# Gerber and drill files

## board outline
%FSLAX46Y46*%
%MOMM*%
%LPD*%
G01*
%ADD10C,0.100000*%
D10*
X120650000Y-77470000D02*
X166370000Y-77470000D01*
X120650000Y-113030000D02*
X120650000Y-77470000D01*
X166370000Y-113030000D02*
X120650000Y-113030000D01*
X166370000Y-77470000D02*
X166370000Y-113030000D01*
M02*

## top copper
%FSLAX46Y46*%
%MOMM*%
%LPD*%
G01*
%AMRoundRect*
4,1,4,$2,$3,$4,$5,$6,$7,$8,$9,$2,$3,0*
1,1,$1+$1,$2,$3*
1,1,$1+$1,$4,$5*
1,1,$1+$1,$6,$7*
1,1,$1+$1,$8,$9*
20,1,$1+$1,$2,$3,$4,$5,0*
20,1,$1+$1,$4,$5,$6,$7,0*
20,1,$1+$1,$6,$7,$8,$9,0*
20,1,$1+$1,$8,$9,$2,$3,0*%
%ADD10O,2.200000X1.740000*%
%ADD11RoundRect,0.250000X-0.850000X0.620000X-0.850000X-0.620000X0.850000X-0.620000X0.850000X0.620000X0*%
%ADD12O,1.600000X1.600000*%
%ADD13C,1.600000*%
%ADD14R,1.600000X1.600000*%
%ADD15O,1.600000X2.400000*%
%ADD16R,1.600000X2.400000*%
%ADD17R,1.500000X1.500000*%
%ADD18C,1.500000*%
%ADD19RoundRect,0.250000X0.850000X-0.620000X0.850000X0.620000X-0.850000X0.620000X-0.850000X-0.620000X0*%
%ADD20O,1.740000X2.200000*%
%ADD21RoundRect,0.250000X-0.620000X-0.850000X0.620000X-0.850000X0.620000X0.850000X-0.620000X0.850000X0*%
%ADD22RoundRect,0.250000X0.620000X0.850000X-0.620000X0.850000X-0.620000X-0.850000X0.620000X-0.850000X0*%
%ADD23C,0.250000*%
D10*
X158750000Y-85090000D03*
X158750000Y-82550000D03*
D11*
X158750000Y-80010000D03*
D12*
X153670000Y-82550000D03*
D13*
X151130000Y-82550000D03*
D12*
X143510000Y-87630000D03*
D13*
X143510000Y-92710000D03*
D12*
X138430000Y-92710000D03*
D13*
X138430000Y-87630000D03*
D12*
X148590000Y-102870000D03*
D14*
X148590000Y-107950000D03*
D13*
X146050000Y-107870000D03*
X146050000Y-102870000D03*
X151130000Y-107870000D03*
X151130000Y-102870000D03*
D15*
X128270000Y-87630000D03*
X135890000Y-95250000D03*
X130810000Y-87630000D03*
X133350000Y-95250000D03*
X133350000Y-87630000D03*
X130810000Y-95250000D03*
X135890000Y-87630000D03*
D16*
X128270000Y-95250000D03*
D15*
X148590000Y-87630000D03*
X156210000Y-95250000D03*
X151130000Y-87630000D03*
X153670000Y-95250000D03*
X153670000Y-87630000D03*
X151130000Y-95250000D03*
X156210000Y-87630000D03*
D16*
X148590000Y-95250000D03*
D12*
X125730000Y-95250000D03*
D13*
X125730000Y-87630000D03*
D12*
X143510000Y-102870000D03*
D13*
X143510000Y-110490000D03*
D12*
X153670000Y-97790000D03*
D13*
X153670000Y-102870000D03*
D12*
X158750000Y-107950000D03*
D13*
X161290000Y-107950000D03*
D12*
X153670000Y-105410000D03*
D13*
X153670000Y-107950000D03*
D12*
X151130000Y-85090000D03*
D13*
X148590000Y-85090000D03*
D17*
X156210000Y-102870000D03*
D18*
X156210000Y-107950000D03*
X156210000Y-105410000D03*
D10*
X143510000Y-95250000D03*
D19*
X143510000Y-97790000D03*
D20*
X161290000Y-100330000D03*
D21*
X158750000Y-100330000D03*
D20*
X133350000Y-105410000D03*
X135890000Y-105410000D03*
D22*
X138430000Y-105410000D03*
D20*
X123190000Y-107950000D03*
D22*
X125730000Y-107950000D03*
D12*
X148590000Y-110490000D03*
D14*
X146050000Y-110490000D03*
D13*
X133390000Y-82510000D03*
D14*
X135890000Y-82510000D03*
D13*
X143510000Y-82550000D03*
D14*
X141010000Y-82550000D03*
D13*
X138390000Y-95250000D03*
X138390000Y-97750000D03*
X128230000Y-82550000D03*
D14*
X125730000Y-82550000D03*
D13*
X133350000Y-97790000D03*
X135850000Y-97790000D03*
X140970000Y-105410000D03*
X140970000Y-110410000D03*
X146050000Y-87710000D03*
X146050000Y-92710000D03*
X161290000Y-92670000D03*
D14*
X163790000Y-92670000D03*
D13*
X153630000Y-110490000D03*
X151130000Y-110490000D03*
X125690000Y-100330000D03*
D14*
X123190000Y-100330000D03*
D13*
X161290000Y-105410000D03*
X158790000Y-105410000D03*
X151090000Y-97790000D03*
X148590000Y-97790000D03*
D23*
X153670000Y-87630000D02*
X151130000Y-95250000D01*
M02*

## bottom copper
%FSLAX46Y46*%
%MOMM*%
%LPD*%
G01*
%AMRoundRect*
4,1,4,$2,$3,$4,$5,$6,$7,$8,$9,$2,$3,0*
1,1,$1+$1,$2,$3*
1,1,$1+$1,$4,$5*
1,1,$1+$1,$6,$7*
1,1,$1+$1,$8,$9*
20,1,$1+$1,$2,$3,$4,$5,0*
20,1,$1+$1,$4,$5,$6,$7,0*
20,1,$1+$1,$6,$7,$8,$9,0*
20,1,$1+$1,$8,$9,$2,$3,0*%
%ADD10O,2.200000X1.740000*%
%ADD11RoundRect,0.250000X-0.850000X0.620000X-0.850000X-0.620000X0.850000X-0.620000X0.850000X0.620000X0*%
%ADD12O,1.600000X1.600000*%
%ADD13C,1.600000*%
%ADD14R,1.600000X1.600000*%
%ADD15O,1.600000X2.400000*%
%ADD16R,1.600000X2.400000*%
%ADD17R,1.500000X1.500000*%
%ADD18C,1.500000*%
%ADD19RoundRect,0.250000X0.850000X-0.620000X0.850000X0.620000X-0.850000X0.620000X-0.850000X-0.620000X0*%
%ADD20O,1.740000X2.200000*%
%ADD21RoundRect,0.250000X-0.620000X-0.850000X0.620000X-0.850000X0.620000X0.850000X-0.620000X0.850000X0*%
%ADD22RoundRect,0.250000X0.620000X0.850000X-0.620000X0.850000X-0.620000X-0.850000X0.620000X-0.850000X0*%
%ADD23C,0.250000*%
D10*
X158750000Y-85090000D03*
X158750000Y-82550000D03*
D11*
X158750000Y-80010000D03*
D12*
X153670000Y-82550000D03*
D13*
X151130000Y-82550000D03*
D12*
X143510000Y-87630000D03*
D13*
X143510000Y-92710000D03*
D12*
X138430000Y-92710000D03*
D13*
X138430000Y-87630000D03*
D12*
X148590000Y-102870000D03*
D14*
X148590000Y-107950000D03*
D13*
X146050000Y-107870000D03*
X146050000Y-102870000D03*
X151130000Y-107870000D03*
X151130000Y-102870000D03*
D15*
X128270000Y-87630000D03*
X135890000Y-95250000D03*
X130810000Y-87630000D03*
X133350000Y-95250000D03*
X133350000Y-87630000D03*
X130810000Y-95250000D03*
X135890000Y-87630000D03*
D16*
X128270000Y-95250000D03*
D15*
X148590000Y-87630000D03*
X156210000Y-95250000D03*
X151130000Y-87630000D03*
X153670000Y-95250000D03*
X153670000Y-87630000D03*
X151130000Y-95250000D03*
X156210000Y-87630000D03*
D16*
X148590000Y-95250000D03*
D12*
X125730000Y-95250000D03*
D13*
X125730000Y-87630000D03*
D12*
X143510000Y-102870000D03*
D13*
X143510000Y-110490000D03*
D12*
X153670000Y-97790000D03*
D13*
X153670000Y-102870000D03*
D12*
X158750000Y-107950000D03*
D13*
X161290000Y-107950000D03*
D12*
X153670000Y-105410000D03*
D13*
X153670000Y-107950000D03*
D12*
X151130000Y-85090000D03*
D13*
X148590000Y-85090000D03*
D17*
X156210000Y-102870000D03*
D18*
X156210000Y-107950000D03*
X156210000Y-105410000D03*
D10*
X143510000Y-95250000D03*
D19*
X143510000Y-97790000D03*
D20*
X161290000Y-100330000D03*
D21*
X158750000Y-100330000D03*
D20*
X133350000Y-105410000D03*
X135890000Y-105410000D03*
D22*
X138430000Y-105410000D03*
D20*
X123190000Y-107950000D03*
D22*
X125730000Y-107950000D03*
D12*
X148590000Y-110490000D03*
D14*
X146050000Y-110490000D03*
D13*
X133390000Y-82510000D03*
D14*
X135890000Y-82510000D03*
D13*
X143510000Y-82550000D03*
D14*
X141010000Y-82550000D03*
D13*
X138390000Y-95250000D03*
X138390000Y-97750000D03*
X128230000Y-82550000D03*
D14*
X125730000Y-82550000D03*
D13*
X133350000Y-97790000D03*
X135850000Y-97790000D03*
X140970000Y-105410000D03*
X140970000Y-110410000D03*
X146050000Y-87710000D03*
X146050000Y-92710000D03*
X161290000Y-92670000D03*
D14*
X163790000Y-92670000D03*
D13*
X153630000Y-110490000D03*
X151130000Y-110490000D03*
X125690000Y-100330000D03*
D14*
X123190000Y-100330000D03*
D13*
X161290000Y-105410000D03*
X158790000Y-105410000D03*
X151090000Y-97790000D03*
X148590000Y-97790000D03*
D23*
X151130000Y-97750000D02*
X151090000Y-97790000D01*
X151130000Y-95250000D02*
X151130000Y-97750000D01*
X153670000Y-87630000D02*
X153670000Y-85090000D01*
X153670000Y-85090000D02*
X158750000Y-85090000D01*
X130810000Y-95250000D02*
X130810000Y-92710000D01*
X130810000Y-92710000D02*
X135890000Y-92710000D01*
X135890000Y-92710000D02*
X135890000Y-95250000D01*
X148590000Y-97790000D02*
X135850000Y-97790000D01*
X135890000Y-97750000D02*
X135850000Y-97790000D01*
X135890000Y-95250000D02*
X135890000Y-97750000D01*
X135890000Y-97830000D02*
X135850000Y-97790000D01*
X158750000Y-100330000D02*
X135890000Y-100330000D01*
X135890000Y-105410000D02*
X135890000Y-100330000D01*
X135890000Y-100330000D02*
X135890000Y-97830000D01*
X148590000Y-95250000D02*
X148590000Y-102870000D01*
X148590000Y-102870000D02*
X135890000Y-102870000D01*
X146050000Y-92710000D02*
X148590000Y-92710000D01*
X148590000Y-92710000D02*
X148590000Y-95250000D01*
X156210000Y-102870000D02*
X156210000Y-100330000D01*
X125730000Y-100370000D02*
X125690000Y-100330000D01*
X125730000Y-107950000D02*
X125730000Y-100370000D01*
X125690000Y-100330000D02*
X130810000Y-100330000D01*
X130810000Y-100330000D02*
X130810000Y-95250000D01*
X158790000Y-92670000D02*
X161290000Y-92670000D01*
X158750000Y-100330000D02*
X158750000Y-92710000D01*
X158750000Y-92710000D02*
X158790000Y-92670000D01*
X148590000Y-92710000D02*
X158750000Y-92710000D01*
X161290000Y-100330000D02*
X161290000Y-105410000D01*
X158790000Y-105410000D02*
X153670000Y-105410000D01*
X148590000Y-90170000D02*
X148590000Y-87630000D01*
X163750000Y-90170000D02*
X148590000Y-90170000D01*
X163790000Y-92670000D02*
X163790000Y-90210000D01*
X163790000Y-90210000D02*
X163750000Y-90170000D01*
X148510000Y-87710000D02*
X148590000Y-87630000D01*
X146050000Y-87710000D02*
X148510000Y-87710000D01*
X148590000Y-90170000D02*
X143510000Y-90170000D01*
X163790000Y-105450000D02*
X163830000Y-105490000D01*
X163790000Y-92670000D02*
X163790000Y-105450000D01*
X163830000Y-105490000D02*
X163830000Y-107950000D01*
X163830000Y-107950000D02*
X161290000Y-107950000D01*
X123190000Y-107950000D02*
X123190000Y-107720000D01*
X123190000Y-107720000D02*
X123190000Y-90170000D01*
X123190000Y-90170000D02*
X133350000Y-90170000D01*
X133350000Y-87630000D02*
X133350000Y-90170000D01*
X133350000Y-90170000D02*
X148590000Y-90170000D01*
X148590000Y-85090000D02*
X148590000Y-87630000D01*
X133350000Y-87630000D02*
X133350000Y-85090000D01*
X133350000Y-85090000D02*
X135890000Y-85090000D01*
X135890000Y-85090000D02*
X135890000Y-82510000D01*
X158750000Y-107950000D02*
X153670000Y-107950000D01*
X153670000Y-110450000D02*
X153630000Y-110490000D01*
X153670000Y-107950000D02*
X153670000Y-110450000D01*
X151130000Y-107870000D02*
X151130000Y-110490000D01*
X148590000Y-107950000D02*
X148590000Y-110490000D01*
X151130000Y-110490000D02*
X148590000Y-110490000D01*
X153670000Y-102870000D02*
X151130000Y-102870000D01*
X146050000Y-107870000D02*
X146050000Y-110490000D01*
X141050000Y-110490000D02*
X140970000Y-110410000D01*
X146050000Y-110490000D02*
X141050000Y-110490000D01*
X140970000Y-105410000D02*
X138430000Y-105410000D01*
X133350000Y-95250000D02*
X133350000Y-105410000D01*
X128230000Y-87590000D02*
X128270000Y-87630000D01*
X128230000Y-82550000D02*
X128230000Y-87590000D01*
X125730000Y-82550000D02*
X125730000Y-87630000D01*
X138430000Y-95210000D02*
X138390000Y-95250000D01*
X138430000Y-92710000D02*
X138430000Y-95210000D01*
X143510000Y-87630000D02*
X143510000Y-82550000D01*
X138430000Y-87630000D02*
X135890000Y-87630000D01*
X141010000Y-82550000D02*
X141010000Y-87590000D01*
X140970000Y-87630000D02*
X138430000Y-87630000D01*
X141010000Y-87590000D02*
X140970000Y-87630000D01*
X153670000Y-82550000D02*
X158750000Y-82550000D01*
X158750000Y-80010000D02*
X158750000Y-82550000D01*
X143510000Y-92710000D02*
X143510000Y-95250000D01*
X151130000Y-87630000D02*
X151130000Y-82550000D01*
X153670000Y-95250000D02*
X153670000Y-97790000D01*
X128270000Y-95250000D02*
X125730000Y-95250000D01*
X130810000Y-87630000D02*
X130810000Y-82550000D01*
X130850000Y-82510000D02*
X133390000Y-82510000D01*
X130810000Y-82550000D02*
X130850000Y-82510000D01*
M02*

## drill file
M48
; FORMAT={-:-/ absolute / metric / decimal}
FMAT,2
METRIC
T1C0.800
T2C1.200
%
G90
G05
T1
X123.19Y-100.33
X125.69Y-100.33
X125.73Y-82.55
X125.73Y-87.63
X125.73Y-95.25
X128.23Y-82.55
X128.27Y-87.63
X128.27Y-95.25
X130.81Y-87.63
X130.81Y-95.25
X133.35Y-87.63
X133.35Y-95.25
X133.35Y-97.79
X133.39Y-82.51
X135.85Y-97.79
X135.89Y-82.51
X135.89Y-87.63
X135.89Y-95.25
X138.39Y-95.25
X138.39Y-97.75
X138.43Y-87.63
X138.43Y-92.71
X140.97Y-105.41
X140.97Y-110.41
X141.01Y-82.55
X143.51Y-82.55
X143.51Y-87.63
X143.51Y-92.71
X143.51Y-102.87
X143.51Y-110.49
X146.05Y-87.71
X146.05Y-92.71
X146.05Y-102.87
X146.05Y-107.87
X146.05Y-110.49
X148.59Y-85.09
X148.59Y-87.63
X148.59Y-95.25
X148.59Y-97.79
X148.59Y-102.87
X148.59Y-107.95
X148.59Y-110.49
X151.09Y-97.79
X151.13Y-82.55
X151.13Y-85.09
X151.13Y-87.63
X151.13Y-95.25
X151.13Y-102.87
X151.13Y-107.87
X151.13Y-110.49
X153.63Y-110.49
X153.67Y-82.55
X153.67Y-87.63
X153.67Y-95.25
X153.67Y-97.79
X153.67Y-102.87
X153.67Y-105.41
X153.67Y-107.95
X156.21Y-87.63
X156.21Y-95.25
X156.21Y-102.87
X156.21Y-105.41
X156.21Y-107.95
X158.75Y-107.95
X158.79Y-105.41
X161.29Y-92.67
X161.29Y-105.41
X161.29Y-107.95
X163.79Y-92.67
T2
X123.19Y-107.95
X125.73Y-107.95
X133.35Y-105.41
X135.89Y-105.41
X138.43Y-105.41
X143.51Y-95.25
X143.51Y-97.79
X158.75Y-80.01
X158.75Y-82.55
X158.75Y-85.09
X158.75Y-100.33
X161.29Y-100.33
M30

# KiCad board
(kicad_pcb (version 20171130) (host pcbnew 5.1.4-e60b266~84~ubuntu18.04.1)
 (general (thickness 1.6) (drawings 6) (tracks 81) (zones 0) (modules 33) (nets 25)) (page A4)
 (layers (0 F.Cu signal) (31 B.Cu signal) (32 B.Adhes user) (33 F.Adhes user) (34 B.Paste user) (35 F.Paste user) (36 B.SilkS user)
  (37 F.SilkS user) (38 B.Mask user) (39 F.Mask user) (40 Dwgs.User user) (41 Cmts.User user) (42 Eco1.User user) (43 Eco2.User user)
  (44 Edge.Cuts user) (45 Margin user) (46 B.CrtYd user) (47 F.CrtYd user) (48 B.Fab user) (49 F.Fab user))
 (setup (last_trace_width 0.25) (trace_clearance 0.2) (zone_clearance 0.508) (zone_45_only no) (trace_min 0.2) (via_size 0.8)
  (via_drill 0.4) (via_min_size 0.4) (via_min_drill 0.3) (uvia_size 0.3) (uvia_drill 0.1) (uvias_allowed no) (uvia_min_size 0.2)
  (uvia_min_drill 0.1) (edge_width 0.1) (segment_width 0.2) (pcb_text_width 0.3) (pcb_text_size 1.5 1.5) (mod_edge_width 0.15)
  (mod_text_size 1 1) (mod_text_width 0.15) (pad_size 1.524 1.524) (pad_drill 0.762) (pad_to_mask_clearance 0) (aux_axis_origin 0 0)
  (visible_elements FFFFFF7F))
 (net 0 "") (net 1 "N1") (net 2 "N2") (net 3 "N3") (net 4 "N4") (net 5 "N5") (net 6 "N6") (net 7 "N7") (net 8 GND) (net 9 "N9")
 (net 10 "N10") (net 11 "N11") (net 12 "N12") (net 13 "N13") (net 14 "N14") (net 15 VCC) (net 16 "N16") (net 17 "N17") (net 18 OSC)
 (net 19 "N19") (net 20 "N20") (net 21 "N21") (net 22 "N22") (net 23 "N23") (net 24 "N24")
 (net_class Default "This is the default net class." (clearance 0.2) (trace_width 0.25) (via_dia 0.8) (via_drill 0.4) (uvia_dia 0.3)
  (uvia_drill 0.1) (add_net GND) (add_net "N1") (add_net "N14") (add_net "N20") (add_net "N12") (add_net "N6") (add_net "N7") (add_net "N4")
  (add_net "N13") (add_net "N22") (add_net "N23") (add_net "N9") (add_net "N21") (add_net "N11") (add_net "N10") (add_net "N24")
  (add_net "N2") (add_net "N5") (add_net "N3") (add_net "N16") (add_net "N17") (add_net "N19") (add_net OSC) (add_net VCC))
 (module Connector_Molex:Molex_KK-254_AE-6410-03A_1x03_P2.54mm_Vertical (layer F.Cu) (at 158.75 80.01 270)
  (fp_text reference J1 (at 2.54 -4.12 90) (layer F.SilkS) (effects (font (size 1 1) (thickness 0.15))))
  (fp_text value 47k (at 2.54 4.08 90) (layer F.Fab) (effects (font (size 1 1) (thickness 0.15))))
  (pad 3 thru_hole oval (at 5.08 0 270) (size 1.74 2.2) (drill 1.2) (layers *.Cu *.Mask) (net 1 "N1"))
  (pad 2 thru_hole oval (at 2.54 0 270) (size 1.74 2.2) (drill 1.2) (layers *.Cu *.Mask) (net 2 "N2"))
  (pad 1 thru_hole roundrect (at 0 0 270) (size 1.74 2.2) (drill 1.2) (layers *.Cu *.Mask) (roundrect_rratio 0.143678) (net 2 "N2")))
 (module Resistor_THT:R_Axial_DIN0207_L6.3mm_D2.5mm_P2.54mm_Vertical (layer F.Cu) (at 151.13 82.55)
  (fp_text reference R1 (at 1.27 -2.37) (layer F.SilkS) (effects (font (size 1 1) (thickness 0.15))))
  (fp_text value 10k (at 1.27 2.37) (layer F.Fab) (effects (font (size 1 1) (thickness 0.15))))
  (pad 2 thru_hole oval (at 2.54 0) (size 1.6 1.6) (drill 0.8) (layers *.Cu *.Mask) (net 2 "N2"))
  (pad 1 thru_hole circle (at 0 0) (size 1.6 1.6) (drill 0.8) (layers *.Cu *.Mask) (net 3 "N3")))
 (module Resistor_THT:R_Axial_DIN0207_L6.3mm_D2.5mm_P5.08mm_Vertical (layer F.Cu) (at 143.51 92.71 90)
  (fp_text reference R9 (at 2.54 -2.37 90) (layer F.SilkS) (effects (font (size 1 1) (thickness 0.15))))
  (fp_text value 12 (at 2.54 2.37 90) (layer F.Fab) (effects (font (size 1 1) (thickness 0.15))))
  (pad 2 thru_hole oval (at 5.08 0 90) (size 1.6 1.6) (drill 0.8) (layers *.Cu *.Mask) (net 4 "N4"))
  (pad 1 thru_hole circle (at 0 0 90) (size 1.6 1.6) (drill 0.8) (layers *.Cu *.Mask) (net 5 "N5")))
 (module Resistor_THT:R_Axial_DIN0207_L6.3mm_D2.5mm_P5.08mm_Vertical (layer F.Cu) (at 138.43 87.63 270)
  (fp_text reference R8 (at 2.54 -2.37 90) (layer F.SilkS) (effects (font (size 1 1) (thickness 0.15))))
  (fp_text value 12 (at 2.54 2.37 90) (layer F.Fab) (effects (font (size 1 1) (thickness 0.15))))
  (pad 2 thru_hole oval (at 5.08 0 270) (size 1.6 1.6) (drill 0.8) (layers *.Cu *.Mask) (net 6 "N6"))
  (pad 1 thru_hole circle (at 0 0 270) (size 1.6 1.6) (drill 0.8) (layers *.Cu *.Mask) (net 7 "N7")))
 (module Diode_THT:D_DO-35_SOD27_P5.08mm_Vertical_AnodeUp (layer F.Cu) (at 148.59 107.95 90)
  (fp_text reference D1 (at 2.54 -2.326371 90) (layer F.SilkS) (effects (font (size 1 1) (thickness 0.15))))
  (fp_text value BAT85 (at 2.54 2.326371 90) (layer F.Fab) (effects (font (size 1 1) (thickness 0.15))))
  (pad 2 thru_hole oval (at 5.08 0 90) (size 1.6 1.6) (drill 0.8) (layers *.Cu *.Mask) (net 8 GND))
  (pad 1 thru_hole rect (at 0 0 90) (size 1.6 1.6) (drill 0.8) (layers *.Cu *.Mask) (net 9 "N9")))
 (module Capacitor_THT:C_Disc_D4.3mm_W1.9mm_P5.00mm (layer F.Cu) (at 146.05 102.87 270)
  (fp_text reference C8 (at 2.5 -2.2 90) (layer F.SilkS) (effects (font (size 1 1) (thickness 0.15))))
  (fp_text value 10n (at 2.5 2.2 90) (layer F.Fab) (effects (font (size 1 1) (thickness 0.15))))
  (pad 2 thru_hole circle (at 5 0 270) (size 1.6 1.6) (drill 0.8) (layers *.Cu *.Mask) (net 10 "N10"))
  (pad 1 thru_hole circle (at 0 0 270) (size 1.6 1.6) (drill 0.8) (layers *.Cu *.Mask) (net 8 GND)))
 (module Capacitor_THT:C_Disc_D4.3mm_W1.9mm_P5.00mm (layer F.Cu) (at 151.13 102.87 270)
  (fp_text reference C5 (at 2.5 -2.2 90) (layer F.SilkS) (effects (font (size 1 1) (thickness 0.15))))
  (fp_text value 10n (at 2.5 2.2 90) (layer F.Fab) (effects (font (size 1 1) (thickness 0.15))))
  (pad 2 thru_hole circle (at 5 0 270) (size 1.6 1.6) (drill 0.8) (layers *.Cu *.Mask) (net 9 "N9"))
  (pad 1 thru_hole circle (at 0 0 270) (size 1.6 1.6) (drill 0.8) (layers *.Cu *.Mask) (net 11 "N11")))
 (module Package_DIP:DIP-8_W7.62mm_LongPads (layer F.Cu) (at 128.27 95.25 90)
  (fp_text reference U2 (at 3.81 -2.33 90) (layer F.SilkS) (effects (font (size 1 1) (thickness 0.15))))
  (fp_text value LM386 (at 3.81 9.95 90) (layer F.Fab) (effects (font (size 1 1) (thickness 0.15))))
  (pad 8 thru_hole oval (at 7.62 0 90) (size 2.4 1.6) (drill 0.8) (layers *.Cu *.Mask) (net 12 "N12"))
  (pad 4 thru_hole oval (at 0 7.62 90) (size 2.4 1.6) (drill 0.8) (layers *.Cu *.Mask) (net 8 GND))
  (pad 7 thru_hole oval (at 7.62 2.54 90) (size 2.4 1.6) (drill 0.8) (layers *.Cu *.Mask) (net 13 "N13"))
  (pad 3 thru_hole oval (at 0 5.08 90) (size 2.4 1.6) (drill 0.8) (layers *.Cu *.Mask) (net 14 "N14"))
  (pad 6 thru_hole oval (at 7.62 5.08 90) (size 2.4 1.6) (drill 0.8) (layers *.Cu *.Mask) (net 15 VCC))
  (pad 2 thru_hole oval (at 0 2.54 90) (size 2.4 1.6) (drill 0.8) (layers *.Cu *.Mask) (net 8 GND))
  (pad 5 thru_hole oval (at 7.62 7.62 90) (size 2.4 1.6) (drill 0.8) (layers *.Cu *.Mask) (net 7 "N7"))
  (pad 1 thru_hole rect (at 0 0 90) (size 2.4 1.6) (drill 0.8) (layers *.Cu *.Mask) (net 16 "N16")))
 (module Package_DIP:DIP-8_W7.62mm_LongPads (layer F.Cu) (at 148.59 95.25 90)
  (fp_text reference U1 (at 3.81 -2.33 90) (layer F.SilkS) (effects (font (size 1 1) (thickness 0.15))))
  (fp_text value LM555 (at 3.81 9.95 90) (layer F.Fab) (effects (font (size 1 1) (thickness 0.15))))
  (pad 8 thru_hole oval (at 7.62 0 90) (size 2.4 1.6) (drill 0.8) (layers *.Cu *.Mask) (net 15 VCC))
  (pad 4 thru_hole oval (at 0 7.62 90) (size 2.4 1.6) (drill 0.8) (layers *.Cu *.Mask) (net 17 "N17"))
  (pad 7 thru_hole oval (at 7.62 2.54 90) (size 2.4 1.6) (drill 0.8) (layers *.Cu *.Mask) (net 3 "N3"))
  (pad 3 thru_hole oval (at 0 5.08 90) (size 2.4 1.6) (drill 0.8) (layers *.Cu *.Mask) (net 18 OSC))
  (pad 6 thru_hole oval (at 7.62 5.08 90) (size 2.4 1.6) (drill 0.8) (layers *.Cu *.Mask) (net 1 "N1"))
  (pad 2 thru_hole oval (at 0 2.54 90) (size 2.4 1.6) (drill 0.8) (layers *.Cu *.Mask) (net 1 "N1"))
  (pad 5 thru_hole oval (at 7.62 7.62 90) (size 2.4 1.6) (drill 0.8) (layers *.Cu *.Mask) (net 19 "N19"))
  (pad 1 thru_hole rect (at 0 0 90) (size 2.4 1.6) (drill 0.8) (layers *.Cu *.Mask) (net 8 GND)))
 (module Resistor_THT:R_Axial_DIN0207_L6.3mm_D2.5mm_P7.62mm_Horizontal (layer F.Cu) (at 125.73 87.63 270)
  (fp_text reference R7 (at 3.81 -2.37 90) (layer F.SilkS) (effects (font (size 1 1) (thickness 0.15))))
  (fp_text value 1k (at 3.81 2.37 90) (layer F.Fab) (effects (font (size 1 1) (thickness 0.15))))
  (pad 2 thru_hole oval (at 7.62 0 270) (size 1.6 1.6) (drill 0.8) (layers *.Cu *.Mask) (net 16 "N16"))
  (pad 1 thru_hole circle (at 0 0 270) (size 1.6 1.6) (drill 0.8) (layers *.Cu *.Mask) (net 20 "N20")))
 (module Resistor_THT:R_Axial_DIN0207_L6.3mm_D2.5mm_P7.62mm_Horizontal (layer F.Cu) (at 143.51 110.49 90)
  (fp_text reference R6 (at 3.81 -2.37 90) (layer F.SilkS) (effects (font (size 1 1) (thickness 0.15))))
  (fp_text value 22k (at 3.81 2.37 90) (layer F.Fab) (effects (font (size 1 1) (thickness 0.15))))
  (pad 2 thru_hole oval (at 7.62 0 90) (size 1.6 1.6) (drill 0.8) (layers *.Cu *.Mask) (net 8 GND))
  (pad 1 thru_hole circle (at 0 0 90) (size 1.6 1.6) (drill 0.8) (layers *.Cu *.Mask) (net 10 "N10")))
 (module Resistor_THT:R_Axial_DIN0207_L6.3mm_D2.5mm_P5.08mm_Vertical (layer F.Cu) (at 153.67 102.87 90)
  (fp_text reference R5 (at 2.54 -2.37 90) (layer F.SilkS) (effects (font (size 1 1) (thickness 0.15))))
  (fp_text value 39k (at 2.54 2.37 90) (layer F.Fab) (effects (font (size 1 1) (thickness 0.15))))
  (pad 2 thru_hole oval (at 5.08 0 90) (size 1.6 1.6) (drill 0.8) (layers *.Cu *.Mask) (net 18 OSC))
  (pad 1 thru_hole circle (at 0 0 90) (size 1.6 1.6) (drill 0.8) (layers *.Cu *.Mask) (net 11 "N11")))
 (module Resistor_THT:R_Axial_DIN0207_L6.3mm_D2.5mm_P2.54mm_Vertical (layer F.Cu) (at 161.29 107.95 180)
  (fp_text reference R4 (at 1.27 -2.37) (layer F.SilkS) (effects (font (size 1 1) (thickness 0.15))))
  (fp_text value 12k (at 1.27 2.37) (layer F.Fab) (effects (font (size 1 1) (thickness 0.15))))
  (pad 2 thru_hole oval (at 2.54 0 180) (size 1.6 1.6) (drill 0.8) (layers *.Cu *.Mask) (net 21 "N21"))
  (pad 1 thru_hole circle (at 0 0 180) (size 1.6 1.6) (drill 0.8) (layers *.Cu *.Mask) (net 15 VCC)))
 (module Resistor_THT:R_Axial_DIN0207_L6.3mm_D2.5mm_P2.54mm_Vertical (layer F.Cu) (at 153.67 107.95 90)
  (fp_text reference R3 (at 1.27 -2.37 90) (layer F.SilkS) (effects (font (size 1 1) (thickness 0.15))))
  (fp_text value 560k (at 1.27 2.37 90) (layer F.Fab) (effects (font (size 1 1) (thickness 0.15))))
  (pad 2 thru_hole oval (at 2.54 0 90) (size 1.6 1.6) (drill 0.8) (layers *.Cu *.Mask) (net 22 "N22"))
  (pad 1 thru_hole circle (at 0 0 90) (size 1.6 1.6) (drill 0.8) (layers *.Cu *.Mask) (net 21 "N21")))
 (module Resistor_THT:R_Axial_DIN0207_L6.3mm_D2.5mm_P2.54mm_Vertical (layer F.Cu) (at 148.59 85.09)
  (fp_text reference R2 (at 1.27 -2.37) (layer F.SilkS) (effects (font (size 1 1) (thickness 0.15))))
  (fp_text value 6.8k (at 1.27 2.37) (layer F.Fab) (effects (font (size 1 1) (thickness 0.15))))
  (pad 2 thru_hole oval (at 2.54 0) (size 1.6 1.6) (drill 0.8) (layers *.Cu *.Mask) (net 3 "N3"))
  (pad 1 thru_hole circle (at 0 0) (size 1.6 1.6) (drill 0.8) (layers *.Cu *.Mask) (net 15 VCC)))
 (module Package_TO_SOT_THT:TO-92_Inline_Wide (layer F.Cu) (at 156.21 102.87 270)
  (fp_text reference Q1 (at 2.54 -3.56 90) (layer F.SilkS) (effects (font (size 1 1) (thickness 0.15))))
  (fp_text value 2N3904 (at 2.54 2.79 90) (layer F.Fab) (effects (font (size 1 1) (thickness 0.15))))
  (pad 1 thru_hole rect (at 0 0) (size 1.5 1.5) (drill 0.8) (layers *.Cu *.Mask) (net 8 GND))
  (pad 3 thru_hole circle (at 5.08 0) (size 1.5 1.5) (drill 0.8) (layers *.Cu *.Mask) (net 21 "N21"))
  (pad 2 thru_hole circle (at 2.54 0) (size 1.5 1.5) (drill 0.8) (layers *.Cu *.Mask) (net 22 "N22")))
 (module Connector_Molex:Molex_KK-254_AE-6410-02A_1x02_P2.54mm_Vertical (layer F.Cu) (at 143.51 97.79 90)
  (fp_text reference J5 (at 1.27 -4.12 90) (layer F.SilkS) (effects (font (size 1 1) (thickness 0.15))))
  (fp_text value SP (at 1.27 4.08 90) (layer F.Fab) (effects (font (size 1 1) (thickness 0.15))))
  (pad 2 thru_hole oval (at 2.54 0 90) (size 1.74 2.2) (drill 1.2) (layers *.Cu *.Mask) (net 5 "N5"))
  (pad 1 thru_hole roundrect (at 0 0 90) (size 1.74 2.2) (drill 1.2) (layers *.Cu *.Mask) (roundrect_rratio 0.143678) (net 8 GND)))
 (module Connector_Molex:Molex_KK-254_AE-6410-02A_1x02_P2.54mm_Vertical (layer F.Cu) (at 158.75 100.33)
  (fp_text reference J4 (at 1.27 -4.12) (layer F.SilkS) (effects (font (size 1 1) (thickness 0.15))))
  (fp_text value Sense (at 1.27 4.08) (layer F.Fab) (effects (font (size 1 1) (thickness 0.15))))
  (pad 2 thru_hole oval (at 2.54 0) (size 1.74 2.2) (drill 1.2) (layers *.Cu *.Mask) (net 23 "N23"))
  (pad 1 thru_hole roundrect (at 0 0) (size 1.74 2.2) (drill 1.2) (layers *.Cu *.Mask) (roundrect_rratio 0.143678) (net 8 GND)))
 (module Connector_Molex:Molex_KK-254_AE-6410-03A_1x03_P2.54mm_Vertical (layer F.Cu) (at 138.43 105.41 180)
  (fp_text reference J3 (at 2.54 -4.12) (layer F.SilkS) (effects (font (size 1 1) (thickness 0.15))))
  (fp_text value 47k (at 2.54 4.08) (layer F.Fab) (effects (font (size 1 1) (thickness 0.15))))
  (pad 3 thru_hole oval (at 5.08 0 180) (size 1.74 2.2) (drill 1.2) (layers *.Cu *.Mask) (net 14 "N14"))
  (pad 2 thru_hole oval (at 2.54 0 180) (size 1.74 2.2) (drill 1.2) (layers *.Cu *.Mask) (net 8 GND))
  (pad 1 thru_hole roundrect (at 0 0 180) (size 1.74 2.2) (drill 1.2) (layers *.Cu *.Mask) (roundrect_rratio 0.143678) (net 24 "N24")))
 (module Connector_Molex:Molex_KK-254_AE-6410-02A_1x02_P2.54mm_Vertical (layer F.Cu) (at 125.73 107.95 180)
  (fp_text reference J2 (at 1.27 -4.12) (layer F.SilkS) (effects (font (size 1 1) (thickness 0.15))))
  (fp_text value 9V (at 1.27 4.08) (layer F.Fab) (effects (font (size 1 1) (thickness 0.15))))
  (pad 2 thru_hole oval (at 2.54 0 180) (size 1.74 2.2) (drill 1.2) (layers *.Cu *.Mask) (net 15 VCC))
  (pad 1 thru_hole roundrect (at 0 0 180) (size 1.74 2.2) (drill 1.2) (layers *.Cu *.Mask) (roundrect_rratio 0.143678) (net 8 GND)))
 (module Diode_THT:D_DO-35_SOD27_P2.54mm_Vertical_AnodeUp (layer F.Cu) (at 146.05 110.49)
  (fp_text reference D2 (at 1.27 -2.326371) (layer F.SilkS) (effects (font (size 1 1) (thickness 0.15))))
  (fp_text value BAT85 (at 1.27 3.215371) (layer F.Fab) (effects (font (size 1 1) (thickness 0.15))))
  (pad 2 thru_hole oval (at 2.54 0) (size 1.6 1.6) (drill 0.8) (layers *.Cu *.Mask) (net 9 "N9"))
  (pad 1 thru_hole rect (at 0 0) (size 1.6 1.6) (drill 0.8) (layers *.Cu *.Mask) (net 10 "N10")))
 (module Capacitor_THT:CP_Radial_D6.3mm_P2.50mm (layer F.Cu) (at 135.89 82.51 180)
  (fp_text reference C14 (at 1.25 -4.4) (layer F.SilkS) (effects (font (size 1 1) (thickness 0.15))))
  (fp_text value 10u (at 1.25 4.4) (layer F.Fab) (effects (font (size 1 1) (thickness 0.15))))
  (pad 2 thru_hole circle (at 2.5 0 180) (size 1.6 1.6) (drill 0.8) (layers *.Cu *.Mask) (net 13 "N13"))
  (pad 1 thru_hole rect (at 0 0 180) (size 1.6 1.6) (drill 0.8) (layers *.Cu *.Mask) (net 15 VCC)))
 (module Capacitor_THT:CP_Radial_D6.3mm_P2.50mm (layer F.Cu) (at 141.01 82.55)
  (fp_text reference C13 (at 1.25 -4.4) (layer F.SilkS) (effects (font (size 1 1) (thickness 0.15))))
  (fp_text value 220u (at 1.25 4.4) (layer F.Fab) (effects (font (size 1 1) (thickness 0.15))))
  (pad 2 thru_hole circle (at 2.5 0) (size 1.6 1.6) (drill 0.8) (layers *.Cu *.Mask) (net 4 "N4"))
  (pad 1 thru_hole rect (at 0 0) (size 1.6 1.6) (drill 0.8) (layers *.Cu *.Mask) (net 7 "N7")))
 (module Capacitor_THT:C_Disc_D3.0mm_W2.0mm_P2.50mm (layer F.Cu) (at 138.39 97.75 90)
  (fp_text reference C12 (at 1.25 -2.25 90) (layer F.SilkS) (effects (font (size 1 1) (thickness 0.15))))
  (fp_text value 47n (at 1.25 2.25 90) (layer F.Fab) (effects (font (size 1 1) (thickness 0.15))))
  (pad 2 thru_hole circle (at 2.5 0 90) (size 1.6 1.6) (drill 0.8) (layers *.Cu *.Mask) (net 6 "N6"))
  (pad 1 thru_hole circle (at 0 0 90) (size 1.6 1.6) (drill 0.8) (layers *.Cu *.Mask) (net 8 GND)))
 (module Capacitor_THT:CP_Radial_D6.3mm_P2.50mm (layer F.Cu) (at 125.73 82.55)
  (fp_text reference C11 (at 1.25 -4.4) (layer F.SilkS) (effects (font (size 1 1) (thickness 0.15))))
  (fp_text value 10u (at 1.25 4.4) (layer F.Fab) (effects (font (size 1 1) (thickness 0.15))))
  (pad 2 thru_hole circle (at 2.5 0) (size 1.6 1.6) (drill 0.8) (layers *.Cu *.Mask) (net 12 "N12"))
  (pad 1 thru_hole rect (at 0 0) (size 1.6 1.6) (drill 0.8) (layers *.Cu *.Mask) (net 20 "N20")))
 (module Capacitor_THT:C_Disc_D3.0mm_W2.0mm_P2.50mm (layer F.Cu) (at 135.85 97.79 180)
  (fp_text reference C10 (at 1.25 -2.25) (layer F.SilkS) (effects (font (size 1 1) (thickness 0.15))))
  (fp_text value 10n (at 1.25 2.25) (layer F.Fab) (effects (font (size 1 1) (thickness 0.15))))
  (pad 2 thru_hole circle (at 2.5 0 180) (size 1.6 1.6) (drill 0.8) (layers *.Cu *.Mask) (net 14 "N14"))
  (pad 1 thru_hole circle (at 0 0 180) (size 1.6 1.6) (drill 0.8) (layers *.Cu *.Mask) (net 8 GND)))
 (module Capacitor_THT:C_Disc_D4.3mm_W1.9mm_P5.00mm (layer F.Cu) (at 140.97 110.41 90)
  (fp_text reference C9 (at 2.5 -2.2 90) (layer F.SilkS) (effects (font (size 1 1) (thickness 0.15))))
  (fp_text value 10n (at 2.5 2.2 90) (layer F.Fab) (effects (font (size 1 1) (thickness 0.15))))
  (pad 2 thru_hole circle (at 5 0 90) (size 1.6 1.6) (drill 0.8) (layers *.Cu *.Mask) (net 24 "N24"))
  (pad 1 thru_hole circle (at 0 0 90) (size 1.6 1.6) (drill 0.8) (layers *.Cu *.Mask) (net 10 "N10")))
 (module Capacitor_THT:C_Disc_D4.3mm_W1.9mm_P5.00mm (layer F.Cu) (at 146.05 92.71 90)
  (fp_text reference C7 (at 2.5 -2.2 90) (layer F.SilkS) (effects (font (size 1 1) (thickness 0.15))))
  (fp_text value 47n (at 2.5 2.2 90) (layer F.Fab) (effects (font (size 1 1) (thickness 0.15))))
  (pad 2 thru_hole circle (at 5 0 90) (size 1.6 1.6) (drill 0.8) (layers *.Cu *.Mask) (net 15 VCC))
  (pad 1 thru_hole circle (at 0 0 90) (size 1.6 1.6) (drill 0.8) (layers *.Cu *.Mask) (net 8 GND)))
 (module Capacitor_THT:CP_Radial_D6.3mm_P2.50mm (layer F.Cu) (at 163.79 92.67 180)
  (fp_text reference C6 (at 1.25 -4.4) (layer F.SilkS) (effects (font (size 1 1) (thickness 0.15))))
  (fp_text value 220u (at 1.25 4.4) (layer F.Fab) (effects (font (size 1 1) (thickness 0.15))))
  (pad 2 thru_hole circle (at 2.5 0 180) (size 1.6 1.6) (drill 0.8) (layers *.Cu *.Mask) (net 8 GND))
  (pad 1 thru_hole rect (at 0 0 180) (size 1.6 1.6) (drill 0.8) (layers *.Cu *.Mask) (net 15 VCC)))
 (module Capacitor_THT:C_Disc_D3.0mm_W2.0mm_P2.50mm (layer F.Cu) (at 151.13 110.49)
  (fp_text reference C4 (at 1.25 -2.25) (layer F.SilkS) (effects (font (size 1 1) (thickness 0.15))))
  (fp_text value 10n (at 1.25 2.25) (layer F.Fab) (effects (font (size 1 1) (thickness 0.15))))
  (pad 2 thru_hole circle (at 2.5 0) (size 1.6 1.6) (drill 0.8) (layers *.Cu *.Mask) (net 21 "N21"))
  (pad 1 thru_hole circle (at 0 0) (size 1.6 1.6) (drill 0.8) (layers *.Cu *.Mask) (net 9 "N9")))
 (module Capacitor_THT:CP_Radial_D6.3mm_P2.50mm (layer F.Cu) (at 123.19 100.33)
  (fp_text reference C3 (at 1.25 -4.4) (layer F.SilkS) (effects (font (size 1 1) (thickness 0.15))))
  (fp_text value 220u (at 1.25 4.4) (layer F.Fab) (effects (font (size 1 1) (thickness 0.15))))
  (pad 2 thru_hole circle (at 2.5 0) (size 1.6 1.6) (drill 0.8) (layers *.Cu *.Mask) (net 8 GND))
  (pad 1 thru_hole rect (at 0 0) (size 1.6 1.6) (drill 0.8) (layers *.Cu *.Mask) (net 15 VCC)))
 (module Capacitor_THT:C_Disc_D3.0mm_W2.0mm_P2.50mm (layer F.Cu) (at 158.79 105.41)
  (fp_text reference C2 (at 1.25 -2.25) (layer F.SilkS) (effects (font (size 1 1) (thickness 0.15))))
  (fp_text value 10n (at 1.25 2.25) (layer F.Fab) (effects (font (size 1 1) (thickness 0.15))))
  (pad 2 thru_hole circle (at 2.5 0) (size 1.6 1.6) (drill 0.8) (layers *.Cu *.Mask) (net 23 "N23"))
  (pad 1 thru_hole circle (at 0 0) (size 1.6 1.6) (drill 0.8) (layers *.Cu *.Mask) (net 22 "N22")))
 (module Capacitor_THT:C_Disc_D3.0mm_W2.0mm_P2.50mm (layer F.Cu) (at 148.59 97.79)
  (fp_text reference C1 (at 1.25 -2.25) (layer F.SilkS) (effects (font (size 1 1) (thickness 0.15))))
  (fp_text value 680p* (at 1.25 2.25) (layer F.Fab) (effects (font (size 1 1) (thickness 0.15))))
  (pad 2 thru_hole circle (at 2.5 0) (size 1.6 1.6) (drill 0.8) (layers *.Cu *.Mask) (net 1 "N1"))
  (pad 1 thru_hole circle (at 0 0) (size 1.6 1.6) (drill 0.8) (layers *.Cu *.Mask) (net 8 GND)))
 (gr_line (start 120.65 77.47) (end 166.37 77.47) (layer Edge.Cuts) (width 0.1))
 (gr_line (start 120.65 113.03) (end 120.65 77.47) (layer Edge.Cuts) (width 0.1))
 (gr_line (start 166.37 113.03) (end 120.65 113.03) (layer Edge.Cuts) (width 0.1))
 (gr_line (start 166.37 77.47) (end 166.37 113.03) (layer Edge.Cuts) (width 0.1))
 (segment (start 153.67 87.63) (end 151.13 95.25) (width 0.25) (layer F.Cu) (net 1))
 (segment (start 151.13 97.75) (end 151.09 97.79) (width 0.25) (layer B.Cu) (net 1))
 (segment (start 151.13 95.25) (end 151.13 97.75) (width 0.25) (layer B.Cu) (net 1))
 (segment (start 153.67 87.63) (end 153.67 85.09) (width 0.25) (layer B.Cu) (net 1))
 (segment (start 153.67 85.09) (end 158.75 85.09) (width 0.25) (layer B.Cu) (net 1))
 (segment (start 130.81 95.25) (end 130.81 92.71) (width 0.25) (layer B.Cu) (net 8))
 (segment (start 130.81 92.71) (end 135.89 92.71) (width 0.25) (layer B.Cu) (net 8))
 (segment (start 135.89 92.71) (end 135.89 95.25) (width 0.25) (layer B.Cu) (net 8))
 (segment (start 148.59 97.79) (end 135.85 97.79) (width 0.25) (layer B.Cu) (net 8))
 (segment (start 135.89 97.75) (end 135.85 97.79) (width 0.25) (layer B.Cu) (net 8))
 (segment (start 135.89 95.25) (end 135.89 97.75) (width 0.25) (layer B.Cu) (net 8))
 (segment (start 135.89 97.83) (end 135.85 97.79) (width 0.25) (layer B.Cu) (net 8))
 (segment (start 158.75 100.33) (end 135.89 100.33) (width 0.25) (layer B.Cu) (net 8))
 (segment (start 135.89 105.41) (end 135.89 100.33) (width 0.25) (layer B.Cu) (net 8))
 (segment (start 135.89 100.33) (end 135.89 97.83) (width 0.25) (layer B.Cu) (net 8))
 (segment (start 148.59 95.25) (end 148.59 102.87) (width 0.25) (layer B.Cu) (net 8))
 (segment (start 148.59 102.87) (end 135.89 102.87) (width 0.25) (layer B.Cu) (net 8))
 (segment (start 146.05 92.71) (end 148.59 92.71) (width 0.25) (layer B.Cu) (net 8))
 (segment (start 148.59 92.71) (end 148.59 95.25) (width 0.25) (layer B.Cu) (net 8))
 (segment (start 156.21 102.87) (end 156.21 100.33) (width 0.25) (layer B.Cu) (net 8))
 (segment (start 125.73 100.37) (end 125.69 100.33) (width 0.25) (layer B.Cu) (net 8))
 (segment (start 125.73 107.95) (end 125.73 100.37) (width 0.25) (layer B.Cu) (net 8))
 (segment (start 125.69 100.33) (end 130.81 100.33) (width 0.25) (layer B.Cu) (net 8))
 (segment (start 130.81 100.33) (end 130.81 95.25) (width 0.25) (layer B.Cu) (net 8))
 (segment (start 158.79 92.67) (end 161.29 92.67) (width 0.25) (layer B.Cu) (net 8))
 (segment (start 158.75 100.33) (end 158.75 92.71) (width 0.25) (layer B.Cu) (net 8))
 (segment (start 158.75 92.71) (end 158.79 92.67) (width 0.25) (layer B.Cu) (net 8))
 (segment (start 148.59 92.71) (end 158.75 92.71) (width 0.25) (layer B.Cu) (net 8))
 (segment (start 161.29 100.33) (end 161.29 105.41) (width 0.25) (layer B.Cu) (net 23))
 (segment (start 158.79 105.41) (end 153.67 105.41) (width 0.25) (layer B.Cu) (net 22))
 (segment (start 148.59 90.17) (end 148.59 87.63) (width 0.25) (layer B.Cu) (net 15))
 (segment (start 163.75 90.17) (end 148.59 90.17) (width 0.25) (layer B.Cu) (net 15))
 (segment (start 163.79 92.67) (end 163.79 90.21) (width 0.25) (layer B.Cu) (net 15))
 (segment (start 163.79 90.21) (end 163.75 90.17) (width 0.25) (layer B.Cu) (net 15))
 (segment (start 148.51 87.71) (end 148.59 87.63) (width 0.25) (layer B.Cu) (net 15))
 (segment (start 146.05 87.71) (end 148.51 87.71) (width 0.25) (layer B.Cu) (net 15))
 (segment (start 148.59 90.17) (end 143.51 90.17) (width 0.25) (layer B.Cu) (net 15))
 (segment (start 163.79 105.45) (end 163.83 105.49) (width 0.25) (layer B.Cu) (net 15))
 (segment (start 163.79 92.67) (end 163.79 105.45) (width 0.25) (layer B.Cu) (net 15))
 (segment (start 163.83 105.49) (end 163.83 107.95) (width 0.25) (layer B.Cu) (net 15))
 (segment (start 163.83 107.95) (end 161.29 107.95) (width 0.25) (layer B.Cu) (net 15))
 (segment (start 123.19 107.95) (end 123.19 107.72) (width 0.25) (layer B.Cu) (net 15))
 (segment (start 123.19 107.72) (end 123.19 90.17) (width 0.25) (layer B.Cu) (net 15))
 (segment (start 123.19 90.17) (end 133.35 90.17) (width 0.25) (layer B.Cu) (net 15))
 (segment (start 133.35 87.63) (end 133.35 90.17) (width 0.25) (layer B.Cu) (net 15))
 (segment (start 133.35 90.17) (end 148.59 90.17) (width 0.25) (layer B.Cu) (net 15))
 (segment (start 148.59 85.09) (end 148.59 87.63) (width 0.25) (layer B.Cu) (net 15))
 (segment (start 133.35 87.63) (end 133.35 85.09) (width 0.25) (layer B.Cu) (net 15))
 (segment (start 133.35 85.09) (end 135.89 85.09) (width 0.25) (layer B.Cu) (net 15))
 (segment (start 135.89 85.09) (end 135.89 82.51) (width 0.25) (layer B.Cu) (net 15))
 (segment (start 158.75 107.95) (end 153.67 107.95) (width 0.25) (layer B.Cu) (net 21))
 (segment (start 153.67 110.45) (end 153.63 110.49) (width 0.25) (layer B.Cu) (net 21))
 (segment (start 153.67 107.95) (end 153.67 110.45) (width 0.25) (layer B.Cu) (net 21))
 (segment (start 151.13 107.87) (end 151.13 110.49) (width 0.25) (layer B.Cu) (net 9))
 (segment (start 148.59 107.95) (end 148.59 110.49) (width 0.25) (layer B.Cu) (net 9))
 (segment (start 151.13 110.49) (end 148.59 110.49) (width 0.25) (layer B.Cu) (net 9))
 (segment (start 153.67 102.87) (end 151.13 102.87) (width 0.25) (layer B.Cu) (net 11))
 (segment (start 146.05 107.87) (end 146.05 110.49) (width 0.25) (layer B.Cu) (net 10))
 (segment (start 141.05 110.49) (end 140.97 110.41) (width 0.25) (layer B.Cu) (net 10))
 (segment (start 146.05 110.49) (end 141.05 110.49) (width 0.25) (layer B.Cu) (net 10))
 (segment (start 140.97 105.41) (end 138.43 105.41) (width 0.25) (layer B.Cu) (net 24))
 (segment (start 133.35 95.25) (end 133.35 105.41) (width 0.25) (layer B.Cu) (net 14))
 (segment (start 128.23 87.59) (end 128.27 87.63) (width 0.25) (layer B.Cu) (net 12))
 (segment (start 128.23 82.55) (end 128.23 87.59) (width 0.25) (layer B.Cu) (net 12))
 (segment (start 125.73 82.55) (end 125.73 87.63) (width 0.25) (layer B.Cu) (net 20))
 (segment (start 138.43 95.21) (end 138.39 95.25) (width 0.25) (layer B.Cu) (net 6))
 (segment (start 138.43 92.71) (end 138.43 95.21) (width 0.25) (layer B.Cu) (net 6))
 (segment (start 143.51 87.63) (end 143.51 82.55) (width 0.25) (layer B.Cu) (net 4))
 (segment (start 138.43 87.63) (end 135.89 87.63) (width 0.25) (layer B.Cu) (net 7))
 (segment (start 141.01 82.55) (end 141.01 87.59) (width 0.25) (layer B.Cu) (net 7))
 (segment (start 140.97 87.63) (end 138.43 87.63) (width 0.25) (layer B.Cu) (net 7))
 (segment (start 141.01 87.59) (end 140.97 87.63) (width 0.25) (layer B.Cu) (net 7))
 (segment (start 153.67 82.55) (end 158.75 82.55) (width 0.25) (layer B.Cu) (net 2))
 (segment (start 158.75 80.01) (end 158.75 82.55) (width 0.25) (layer B.Cu) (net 2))
 (segment (start 143.51 92.71) (end 143.51 95.25) (width 0.25) (layer B.Cu) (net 5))
 (segment (start 151.13 87.63) (end 151.13 82.55) (width 0.25) (layer B.Cu) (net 3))
 (segment (start 153.67 95.25) (end 153.67 97.79) (width 0.25) (layer B.Cu) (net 18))
 (segment (start 128.27 95.25) (end 125.73 95.25) (width 0.25) (layer B.Cu) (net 16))
 (segment (start 130.81 87.63) (end 130.81 82.55) (width 0.25) (layer B.Cu) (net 13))
 (segment (start 130.85 82.51) (end 133.39 82.51) (width 0.25) (layer B.Cu) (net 13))
 (segment (start 130.81 82.55) (end 130.85 82.51) (width 0.25) (layer B.Cu) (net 13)))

